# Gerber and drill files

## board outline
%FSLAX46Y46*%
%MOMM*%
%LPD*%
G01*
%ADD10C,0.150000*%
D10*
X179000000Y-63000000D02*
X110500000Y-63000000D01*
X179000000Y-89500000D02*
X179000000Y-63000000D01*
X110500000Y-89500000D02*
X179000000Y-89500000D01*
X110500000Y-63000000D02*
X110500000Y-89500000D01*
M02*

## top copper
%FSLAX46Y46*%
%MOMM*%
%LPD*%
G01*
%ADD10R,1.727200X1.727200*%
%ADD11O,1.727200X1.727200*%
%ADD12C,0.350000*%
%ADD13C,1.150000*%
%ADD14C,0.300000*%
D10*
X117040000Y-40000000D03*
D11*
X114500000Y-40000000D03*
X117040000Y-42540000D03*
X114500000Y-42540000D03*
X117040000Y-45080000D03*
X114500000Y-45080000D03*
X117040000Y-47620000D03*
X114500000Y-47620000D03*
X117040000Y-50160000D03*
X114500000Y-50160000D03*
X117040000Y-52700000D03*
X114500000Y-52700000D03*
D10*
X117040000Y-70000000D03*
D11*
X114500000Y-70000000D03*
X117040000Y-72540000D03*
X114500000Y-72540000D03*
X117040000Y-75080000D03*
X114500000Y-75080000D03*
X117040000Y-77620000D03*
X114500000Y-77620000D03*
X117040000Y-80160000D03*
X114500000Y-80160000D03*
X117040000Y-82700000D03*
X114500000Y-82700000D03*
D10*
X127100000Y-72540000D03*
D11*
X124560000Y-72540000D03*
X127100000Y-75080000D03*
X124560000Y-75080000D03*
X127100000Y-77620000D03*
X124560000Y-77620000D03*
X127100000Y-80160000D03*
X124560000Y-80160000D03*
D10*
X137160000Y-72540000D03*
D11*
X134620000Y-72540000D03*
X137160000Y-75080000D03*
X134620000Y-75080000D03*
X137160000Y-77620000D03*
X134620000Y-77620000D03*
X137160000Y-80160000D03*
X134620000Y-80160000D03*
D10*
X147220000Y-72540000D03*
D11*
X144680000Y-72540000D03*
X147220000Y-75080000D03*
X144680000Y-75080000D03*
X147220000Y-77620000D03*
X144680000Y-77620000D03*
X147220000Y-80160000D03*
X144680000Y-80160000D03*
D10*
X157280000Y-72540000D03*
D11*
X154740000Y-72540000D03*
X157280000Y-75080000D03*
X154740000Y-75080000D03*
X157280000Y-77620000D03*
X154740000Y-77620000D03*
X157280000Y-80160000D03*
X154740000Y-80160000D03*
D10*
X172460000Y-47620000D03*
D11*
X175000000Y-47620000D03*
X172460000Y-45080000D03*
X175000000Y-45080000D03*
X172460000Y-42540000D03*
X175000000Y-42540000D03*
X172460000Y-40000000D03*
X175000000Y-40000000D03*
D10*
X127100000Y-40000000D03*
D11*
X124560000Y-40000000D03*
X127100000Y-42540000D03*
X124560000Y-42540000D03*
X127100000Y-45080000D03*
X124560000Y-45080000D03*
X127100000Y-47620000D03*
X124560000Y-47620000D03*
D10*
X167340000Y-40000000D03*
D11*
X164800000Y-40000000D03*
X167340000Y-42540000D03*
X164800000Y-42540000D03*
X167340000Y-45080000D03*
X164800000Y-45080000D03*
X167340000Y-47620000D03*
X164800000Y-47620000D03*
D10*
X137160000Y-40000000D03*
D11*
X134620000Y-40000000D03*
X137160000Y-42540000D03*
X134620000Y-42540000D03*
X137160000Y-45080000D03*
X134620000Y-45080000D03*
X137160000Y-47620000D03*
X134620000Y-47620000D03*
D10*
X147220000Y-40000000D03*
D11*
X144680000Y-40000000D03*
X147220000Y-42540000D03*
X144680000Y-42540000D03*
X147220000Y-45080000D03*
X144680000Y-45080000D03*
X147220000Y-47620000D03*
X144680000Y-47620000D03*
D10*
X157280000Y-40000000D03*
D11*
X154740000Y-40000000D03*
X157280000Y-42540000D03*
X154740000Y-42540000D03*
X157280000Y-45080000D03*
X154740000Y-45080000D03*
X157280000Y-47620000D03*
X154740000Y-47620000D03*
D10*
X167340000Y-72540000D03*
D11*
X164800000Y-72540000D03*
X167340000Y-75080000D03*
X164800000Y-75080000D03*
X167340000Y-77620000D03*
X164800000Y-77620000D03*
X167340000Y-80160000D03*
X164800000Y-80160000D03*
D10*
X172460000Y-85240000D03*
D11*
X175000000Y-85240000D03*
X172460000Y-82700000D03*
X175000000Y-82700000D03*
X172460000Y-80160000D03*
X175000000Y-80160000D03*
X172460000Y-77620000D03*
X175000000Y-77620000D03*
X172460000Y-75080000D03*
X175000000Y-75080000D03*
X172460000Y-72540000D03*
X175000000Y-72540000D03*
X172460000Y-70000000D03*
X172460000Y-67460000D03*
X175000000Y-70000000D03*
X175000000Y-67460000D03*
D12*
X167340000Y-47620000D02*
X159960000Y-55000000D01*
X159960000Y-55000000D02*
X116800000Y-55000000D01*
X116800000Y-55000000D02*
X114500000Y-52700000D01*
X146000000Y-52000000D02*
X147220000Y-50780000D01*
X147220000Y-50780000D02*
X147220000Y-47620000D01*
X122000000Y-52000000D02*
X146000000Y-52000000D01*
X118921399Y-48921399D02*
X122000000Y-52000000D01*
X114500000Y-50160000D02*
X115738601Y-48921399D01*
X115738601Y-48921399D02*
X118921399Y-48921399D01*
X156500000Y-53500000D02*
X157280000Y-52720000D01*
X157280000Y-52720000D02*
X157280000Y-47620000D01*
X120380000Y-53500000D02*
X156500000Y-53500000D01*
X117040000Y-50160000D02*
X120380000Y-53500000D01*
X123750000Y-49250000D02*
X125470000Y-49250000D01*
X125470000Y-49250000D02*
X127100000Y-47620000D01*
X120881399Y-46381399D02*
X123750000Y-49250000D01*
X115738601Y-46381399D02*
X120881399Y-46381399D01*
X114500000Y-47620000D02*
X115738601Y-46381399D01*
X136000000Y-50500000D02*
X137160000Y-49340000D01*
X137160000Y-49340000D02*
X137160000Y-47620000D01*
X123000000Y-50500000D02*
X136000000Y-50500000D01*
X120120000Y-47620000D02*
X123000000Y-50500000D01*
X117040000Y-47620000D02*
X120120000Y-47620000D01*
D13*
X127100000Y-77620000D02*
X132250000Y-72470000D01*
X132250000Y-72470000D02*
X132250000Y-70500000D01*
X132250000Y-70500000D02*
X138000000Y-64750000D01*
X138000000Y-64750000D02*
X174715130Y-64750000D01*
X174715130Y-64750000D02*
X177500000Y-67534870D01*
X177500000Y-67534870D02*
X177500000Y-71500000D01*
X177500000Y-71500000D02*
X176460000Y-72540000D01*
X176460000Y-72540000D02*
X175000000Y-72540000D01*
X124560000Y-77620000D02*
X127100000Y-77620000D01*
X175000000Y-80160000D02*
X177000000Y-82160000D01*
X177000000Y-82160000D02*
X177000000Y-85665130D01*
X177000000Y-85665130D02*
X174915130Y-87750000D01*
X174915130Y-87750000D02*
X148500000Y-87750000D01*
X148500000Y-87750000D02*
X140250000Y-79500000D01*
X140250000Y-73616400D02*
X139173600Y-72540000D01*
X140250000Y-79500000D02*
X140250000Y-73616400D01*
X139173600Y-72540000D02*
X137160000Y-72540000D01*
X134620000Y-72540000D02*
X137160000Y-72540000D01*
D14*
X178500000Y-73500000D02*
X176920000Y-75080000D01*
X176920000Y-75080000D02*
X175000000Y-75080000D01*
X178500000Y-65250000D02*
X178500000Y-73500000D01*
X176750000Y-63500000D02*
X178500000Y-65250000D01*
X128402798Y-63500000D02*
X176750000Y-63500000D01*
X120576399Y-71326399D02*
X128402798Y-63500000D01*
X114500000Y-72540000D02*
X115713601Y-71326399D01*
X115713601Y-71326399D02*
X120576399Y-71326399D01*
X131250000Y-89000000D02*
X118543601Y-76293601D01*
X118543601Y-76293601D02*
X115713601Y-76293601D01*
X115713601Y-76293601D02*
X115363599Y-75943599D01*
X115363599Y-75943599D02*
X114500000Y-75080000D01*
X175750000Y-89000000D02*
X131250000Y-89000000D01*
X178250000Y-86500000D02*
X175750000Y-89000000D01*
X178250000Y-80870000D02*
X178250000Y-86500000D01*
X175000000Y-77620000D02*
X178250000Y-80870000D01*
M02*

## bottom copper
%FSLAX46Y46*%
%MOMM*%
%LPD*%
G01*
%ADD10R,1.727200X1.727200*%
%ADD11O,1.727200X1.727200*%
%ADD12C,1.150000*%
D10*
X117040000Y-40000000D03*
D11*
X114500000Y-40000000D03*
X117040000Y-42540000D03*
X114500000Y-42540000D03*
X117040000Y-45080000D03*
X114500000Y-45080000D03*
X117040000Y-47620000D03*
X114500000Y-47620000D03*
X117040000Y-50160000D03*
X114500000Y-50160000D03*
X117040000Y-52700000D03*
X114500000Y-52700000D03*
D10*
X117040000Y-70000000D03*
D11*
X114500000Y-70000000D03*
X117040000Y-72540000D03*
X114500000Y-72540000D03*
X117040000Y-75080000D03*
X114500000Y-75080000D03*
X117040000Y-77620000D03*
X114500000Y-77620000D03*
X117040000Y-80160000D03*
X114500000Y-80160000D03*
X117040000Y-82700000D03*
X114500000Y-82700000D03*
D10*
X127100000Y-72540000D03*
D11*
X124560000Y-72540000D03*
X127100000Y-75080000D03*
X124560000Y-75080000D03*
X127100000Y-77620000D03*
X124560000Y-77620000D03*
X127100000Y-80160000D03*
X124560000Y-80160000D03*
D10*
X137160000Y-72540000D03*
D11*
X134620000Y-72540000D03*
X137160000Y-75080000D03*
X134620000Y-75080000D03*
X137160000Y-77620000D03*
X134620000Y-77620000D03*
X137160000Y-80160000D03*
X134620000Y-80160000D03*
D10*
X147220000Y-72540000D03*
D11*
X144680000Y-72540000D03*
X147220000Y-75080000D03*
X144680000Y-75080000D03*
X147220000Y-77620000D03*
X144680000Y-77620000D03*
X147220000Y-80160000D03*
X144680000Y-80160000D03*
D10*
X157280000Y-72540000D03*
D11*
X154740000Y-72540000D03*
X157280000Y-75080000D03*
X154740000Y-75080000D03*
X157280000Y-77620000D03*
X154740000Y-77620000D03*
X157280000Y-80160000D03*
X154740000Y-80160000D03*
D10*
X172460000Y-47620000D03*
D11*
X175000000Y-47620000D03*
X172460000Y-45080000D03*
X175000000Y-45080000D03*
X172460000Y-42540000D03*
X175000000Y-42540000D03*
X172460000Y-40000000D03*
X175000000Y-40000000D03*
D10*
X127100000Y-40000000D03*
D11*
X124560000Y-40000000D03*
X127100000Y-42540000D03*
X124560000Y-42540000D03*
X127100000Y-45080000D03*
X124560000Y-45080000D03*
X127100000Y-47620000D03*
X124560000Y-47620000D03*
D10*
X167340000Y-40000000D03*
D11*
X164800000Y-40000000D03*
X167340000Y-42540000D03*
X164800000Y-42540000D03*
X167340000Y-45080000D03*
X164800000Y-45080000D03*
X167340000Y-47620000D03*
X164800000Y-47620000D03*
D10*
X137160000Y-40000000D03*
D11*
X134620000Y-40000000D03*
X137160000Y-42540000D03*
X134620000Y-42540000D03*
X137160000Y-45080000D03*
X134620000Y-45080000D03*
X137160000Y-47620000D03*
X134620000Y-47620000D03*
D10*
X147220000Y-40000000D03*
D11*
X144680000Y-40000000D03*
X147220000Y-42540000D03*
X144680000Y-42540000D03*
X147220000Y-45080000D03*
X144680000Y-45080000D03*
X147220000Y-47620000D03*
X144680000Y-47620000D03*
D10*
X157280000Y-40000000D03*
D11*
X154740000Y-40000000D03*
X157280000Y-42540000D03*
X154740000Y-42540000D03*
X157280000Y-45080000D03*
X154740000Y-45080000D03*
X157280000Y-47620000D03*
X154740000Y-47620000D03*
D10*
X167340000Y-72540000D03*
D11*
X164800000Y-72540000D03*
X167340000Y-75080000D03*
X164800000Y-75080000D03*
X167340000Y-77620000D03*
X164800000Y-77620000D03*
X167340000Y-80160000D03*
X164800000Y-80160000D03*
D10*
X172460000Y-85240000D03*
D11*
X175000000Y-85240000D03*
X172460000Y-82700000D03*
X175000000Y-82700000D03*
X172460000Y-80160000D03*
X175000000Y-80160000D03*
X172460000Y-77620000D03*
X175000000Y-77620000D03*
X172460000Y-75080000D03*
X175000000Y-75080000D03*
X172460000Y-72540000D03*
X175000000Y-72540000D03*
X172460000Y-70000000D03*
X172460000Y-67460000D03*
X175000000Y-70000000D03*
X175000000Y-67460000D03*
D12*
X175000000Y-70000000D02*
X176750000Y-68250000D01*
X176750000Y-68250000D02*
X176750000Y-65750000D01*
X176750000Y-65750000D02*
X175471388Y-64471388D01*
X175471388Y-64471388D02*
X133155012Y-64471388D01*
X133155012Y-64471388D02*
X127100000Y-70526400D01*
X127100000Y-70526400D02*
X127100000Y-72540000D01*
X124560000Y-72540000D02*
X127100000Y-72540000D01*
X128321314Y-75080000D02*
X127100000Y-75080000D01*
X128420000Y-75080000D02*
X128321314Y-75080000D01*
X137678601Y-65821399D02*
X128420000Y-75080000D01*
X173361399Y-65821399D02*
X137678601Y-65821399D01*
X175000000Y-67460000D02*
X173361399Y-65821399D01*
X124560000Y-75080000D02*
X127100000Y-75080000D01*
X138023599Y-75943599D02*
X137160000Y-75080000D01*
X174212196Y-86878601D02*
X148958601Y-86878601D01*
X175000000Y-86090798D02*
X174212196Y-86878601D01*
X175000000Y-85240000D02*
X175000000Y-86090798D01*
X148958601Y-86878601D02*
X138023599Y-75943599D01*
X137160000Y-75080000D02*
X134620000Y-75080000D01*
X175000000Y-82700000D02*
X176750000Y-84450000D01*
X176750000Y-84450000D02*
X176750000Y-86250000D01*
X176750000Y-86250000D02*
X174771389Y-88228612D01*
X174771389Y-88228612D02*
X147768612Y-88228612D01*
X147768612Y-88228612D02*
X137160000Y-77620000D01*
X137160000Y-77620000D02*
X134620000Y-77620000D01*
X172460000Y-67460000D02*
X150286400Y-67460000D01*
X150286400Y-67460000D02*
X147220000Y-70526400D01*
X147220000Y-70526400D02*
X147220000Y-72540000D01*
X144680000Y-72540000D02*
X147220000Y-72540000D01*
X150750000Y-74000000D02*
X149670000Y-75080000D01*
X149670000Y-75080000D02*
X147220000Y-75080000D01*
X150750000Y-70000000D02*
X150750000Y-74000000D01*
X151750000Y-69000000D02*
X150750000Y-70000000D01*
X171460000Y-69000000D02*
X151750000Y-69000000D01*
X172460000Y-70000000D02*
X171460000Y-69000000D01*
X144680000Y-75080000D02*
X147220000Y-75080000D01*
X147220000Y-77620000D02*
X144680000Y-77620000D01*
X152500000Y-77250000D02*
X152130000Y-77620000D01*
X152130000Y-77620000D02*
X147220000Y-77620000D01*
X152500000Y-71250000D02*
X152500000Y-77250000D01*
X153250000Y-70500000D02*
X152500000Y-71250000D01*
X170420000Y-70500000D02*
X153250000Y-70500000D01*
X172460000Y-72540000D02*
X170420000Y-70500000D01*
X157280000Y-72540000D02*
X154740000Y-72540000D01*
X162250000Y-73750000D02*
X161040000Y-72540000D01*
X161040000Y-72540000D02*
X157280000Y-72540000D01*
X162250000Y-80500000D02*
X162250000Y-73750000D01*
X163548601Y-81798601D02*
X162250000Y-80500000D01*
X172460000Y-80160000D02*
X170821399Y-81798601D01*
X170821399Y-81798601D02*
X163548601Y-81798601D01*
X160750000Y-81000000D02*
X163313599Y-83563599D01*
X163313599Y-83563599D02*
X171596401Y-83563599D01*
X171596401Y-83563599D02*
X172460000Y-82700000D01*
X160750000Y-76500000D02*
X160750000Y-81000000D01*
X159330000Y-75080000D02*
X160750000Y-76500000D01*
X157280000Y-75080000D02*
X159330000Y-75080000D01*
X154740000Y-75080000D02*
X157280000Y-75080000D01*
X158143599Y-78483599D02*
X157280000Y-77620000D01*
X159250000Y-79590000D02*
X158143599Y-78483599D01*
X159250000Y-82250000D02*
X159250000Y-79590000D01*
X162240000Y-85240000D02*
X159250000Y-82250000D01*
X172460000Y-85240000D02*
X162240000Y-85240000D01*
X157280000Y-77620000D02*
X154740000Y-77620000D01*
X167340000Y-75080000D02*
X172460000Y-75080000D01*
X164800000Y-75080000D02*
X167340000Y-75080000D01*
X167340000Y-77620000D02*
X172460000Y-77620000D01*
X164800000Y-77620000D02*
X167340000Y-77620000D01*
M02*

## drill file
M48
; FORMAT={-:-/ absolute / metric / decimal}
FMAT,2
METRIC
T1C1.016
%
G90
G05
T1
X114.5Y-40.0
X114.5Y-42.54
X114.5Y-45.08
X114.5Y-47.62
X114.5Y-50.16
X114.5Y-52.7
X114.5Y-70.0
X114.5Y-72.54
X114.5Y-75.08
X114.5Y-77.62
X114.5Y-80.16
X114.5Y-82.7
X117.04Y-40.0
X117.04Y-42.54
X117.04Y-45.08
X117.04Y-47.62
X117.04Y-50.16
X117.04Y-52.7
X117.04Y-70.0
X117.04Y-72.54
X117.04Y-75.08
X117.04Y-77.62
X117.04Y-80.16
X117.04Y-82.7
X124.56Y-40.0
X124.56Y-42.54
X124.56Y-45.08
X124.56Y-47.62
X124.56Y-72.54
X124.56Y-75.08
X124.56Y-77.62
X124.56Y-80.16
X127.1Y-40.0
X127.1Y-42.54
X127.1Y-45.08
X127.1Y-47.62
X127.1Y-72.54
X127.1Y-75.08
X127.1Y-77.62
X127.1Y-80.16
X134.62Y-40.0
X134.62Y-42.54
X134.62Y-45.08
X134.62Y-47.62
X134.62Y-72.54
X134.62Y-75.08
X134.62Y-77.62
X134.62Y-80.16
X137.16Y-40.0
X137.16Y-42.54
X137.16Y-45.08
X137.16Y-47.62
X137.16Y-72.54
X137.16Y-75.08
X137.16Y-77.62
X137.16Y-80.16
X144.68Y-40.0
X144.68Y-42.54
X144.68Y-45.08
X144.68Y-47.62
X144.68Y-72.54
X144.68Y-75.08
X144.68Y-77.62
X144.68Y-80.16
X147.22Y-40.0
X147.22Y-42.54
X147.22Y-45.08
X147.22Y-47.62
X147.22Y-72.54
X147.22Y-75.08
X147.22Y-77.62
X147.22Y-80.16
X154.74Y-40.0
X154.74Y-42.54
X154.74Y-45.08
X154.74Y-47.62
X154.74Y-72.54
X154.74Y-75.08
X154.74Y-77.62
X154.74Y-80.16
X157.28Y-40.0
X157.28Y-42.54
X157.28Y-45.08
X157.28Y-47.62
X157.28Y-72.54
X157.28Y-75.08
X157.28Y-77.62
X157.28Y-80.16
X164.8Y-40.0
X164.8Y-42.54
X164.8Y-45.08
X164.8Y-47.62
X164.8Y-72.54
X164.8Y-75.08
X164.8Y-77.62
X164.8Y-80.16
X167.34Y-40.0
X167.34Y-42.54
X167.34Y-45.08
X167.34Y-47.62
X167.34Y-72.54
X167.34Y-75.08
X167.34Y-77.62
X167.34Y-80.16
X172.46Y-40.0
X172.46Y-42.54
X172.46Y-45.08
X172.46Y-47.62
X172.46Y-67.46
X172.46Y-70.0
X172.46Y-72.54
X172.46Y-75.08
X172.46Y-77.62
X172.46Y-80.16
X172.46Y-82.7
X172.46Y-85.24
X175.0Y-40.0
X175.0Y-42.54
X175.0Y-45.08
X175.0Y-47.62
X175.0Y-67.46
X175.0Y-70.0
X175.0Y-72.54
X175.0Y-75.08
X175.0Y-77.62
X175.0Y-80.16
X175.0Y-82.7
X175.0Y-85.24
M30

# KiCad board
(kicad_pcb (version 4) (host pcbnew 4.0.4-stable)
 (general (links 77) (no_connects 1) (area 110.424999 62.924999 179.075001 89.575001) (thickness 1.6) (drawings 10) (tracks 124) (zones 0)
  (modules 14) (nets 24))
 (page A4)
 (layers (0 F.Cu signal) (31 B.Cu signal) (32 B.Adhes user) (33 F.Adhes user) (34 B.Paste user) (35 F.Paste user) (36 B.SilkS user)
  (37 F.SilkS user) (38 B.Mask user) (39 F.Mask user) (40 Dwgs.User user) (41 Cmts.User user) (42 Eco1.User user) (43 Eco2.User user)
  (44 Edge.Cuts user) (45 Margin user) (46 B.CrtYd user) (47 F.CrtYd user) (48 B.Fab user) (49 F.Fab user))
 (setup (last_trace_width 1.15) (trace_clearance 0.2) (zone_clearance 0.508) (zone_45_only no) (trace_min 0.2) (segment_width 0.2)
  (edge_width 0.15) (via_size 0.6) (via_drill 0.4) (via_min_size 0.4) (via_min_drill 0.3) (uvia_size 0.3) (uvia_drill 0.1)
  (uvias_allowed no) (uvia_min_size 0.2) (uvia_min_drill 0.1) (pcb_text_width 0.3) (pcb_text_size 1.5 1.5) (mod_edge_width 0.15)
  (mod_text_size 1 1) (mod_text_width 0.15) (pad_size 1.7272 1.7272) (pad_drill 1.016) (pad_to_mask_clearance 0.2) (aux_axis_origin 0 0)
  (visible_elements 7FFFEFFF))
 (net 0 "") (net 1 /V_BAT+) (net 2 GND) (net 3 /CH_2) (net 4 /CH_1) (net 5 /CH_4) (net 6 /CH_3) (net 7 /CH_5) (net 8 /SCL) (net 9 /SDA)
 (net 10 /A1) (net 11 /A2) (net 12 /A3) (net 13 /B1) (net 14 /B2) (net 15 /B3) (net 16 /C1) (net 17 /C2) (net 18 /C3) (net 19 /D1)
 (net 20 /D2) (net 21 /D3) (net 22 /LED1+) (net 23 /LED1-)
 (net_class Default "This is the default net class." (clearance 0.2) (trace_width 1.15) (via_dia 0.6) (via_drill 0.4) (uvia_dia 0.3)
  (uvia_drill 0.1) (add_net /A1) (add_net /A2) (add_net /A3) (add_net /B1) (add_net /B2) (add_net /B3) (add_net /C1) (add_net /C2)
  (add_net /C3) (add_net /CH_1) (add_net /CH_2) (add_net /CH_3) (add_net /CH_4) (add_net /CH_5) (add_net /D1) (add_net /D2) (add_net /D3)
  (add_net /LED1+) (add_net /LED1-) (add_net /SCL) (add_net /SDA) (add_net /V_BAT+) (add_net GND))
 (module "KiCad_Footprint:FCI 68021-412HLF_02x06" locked (layer F.Cu) (at 117.04 40 270)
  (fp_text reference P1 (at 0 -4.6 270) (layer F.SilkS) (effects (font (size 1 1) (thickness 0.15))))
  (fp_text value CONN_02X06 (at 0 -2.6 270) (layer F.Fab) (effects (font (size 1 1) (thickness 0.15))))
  (pad 1 thru_hole rect (at 0 0 270) (size 1.7272 1.7272) (drill 1.016) (layers *.Cu *.Mask F.SilkS) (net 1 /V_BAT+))
  (pad 2 thru_hole oval (at 0 2.54 270) (size 1.7272 1.7272) (drill 1.016) (layers *.Cu *.Mask F.SilkS) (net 1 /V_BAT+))
  (pad 3 thru_hole oval (at 2.54 0 270) (size 1.7272 1.7272) (drill 1.016) (layers *.Cu *.Mask F.SilkS) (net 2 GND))
  (pad 4 thru_hole oval (at 2.54 2.54 270) (size 1.7272 1.7272) (drill 1.016) (layers *.Cu *.Mask F.SilkS) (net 2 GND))
  (pad 5 thru_hole oval (at 5.08 0 270) (size 1.7272 1.7272) (drill 1.016) (layers *.Cu *.Mask F.SilkS) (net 2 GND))
  (pad 6 thru_hole oval (at 5.08 2.54 270) (size 1.7272 1.7272) (drill 1.016) (layers *.Cu *.Mask F.SilkS) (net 2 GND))
  (pad 7 thru_hole oval (at 7.62 0 270) (size 1.7272 1.7272) (drill 1.016) (layers *.Cu *.Mask F.SilkS) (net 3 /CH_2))
  (pad 8 thru_hole oval (at 7.62 2.54 270) (size 1.7272 1.7272) (drill 1.016) (layers *.Cu *.Mask F.SilkS) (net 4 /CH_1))
  (pad 9 thru_hole oval (at 10.16 0 270) (size 1.7272 1.7272) (drill 1.016) (layers *.Cu *.Mask F.SilkS) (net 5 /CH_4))
  (pad 10 thru_hole oval (at 10.16 2.54 270) (size 1.7272 1.7272) (drill 1.016) (layers *.Cu *.Mask F.SilkS) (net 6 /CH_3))
  (pad 11 thru_hole oval (at 12.7 0 270) (size 1.7272 1.7272) (drill 1.016) (layers *.Cu *.Mask F.SilkS))
  (pad 12 thru_hole oval (at 12.7 2.54 270) (size 1.7272 1.7272) (drill 1.016) (layers *.Cu *.Mask F.SilkS) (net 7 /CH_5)))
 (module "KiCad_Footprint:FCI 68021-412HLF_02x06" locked (layer F.Cu) (at 117.04 70 270)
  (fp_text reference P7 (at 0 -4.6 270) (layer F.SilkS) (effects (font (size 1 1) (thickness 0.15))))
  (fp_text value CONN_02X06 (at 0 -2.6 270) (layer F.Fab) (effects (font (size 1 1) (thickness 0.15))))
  (pad 1 thru_hole rect (at 0 0 270) (size 1.7272 1.7272) (drill 1.016) (layers *.Cu *.Mask F.SilkS))
  (pad 2 thru_hole oval (at 0 2.54 270) (size 1.7272 1.7272) (drill 1.016) (layers *.Cu *.Mask F.SilkS))
  (pad 3 thru_hole oval (at 2.54 0 270) (size 1.7272 1.7272) (drill 1.016) (layers *.Cu *.Mask F.SilkS))
  (pad 4 thru_hole oval (at 2.54 2.54 270) (size 1.7272 1.7272) (drill 1.016) (layers *.Cu *.Mask F.SilkS) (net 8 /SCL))
  (pad 5 thru_hole oval (at 5.08 0 270) (size 1.7272 1.7272) (drill 1.016) (layers *.Cu *.Mask F.SilkS))
  (pad 6 thru_hole oval (at 5.08 2.54 270) (size 1.7272 1.7272) (drill 1.016) (layers *.Cu *.Mask F.SilkS) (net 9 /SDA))
  (pad 7 thru_hole oval (at 7.62 0 270) (size 1.7272 1.7272) (drill 1.016) (layers *.Cu *.Mask F.SilkS))
  (pad 8 thru_hole oval (at 7.62 2.54 270) (size 1.7272 1.7272) (drill 1.016) (layers *.Cu *.Mask F.SilkS))
  (pad 9 thru_hole oval (at 10.16 0 270) (size 1.7272 1.7272) (drill 1.016) (layers *.Cu *.Mask F.SilkS))
  (pad 10 thru_hole oval (at 10.16 2.54 270) (size 1.7272 1.7272) (drill 1.016) (layers *.Cu *.Mask F.SilkS))
  (pad 11 thru_hole oval (at 12.7 0 270) (size 1.7272 1.7272) (drill 1.016) (layers *.Cu *.Mask F.SilkS))
  (pad 12 thru_hole oval (at 12.7 2.54 270) (size 1.7272 1.7272) (drill 1.016) (layers *.Cu *.Mask F.SilkS)))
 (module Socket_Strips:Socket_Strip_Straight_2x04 (layer F.Cu) (at 127.1 72.54 270)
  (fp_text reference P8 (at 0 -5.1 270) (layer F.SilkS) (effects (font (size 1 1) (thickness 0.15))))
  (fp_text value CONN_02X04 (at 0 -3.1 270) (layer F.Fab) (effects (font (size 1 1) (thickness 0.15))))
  (pad 1 thru_hole rect (at 0 0 270) (size 1.7272 1.7272) (drill 1.016) (layers *.Cu *.Mask F.SilkS) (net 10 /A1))
  (pad 2 thru_hole oval (at 0 2.54 270) (size 1.7272 1.7272) (drill 1.016) (layers *.Cu *.Mask F.SilkS) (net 10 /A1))
  (pad 3 thru_hole oval (at 2.54 0 270) (size 1.7272 1.7272) (drill 1.016) (layers *.Cu *.Mask F.SilkS) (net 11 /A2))
  (pad 4 thru_hole oval (at 2.54 2.54 270) (size 1.7272 1.7272) (drill 1.016) (layers *.Cu *.Mask F.SilkS) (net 11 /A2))
  (pad 5 thru_hole oval (at 5.08 0 270) (size 1.7272 1.7272) (drill 1.016) (layers *.Cu *.Mask F.SilkS) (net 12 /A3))
  (pad 6 thru_hole oval (at 5.08 2.54 270) (size 1.7272 1.7272) (drill 1.016) (layers *.Cu *.Mask F.SilkS) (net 12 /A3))
  (pad 7 thru_hole oval (at 7.62 0 270) (size 1.7272 1.7272) (drill 1.016) (layers *.Cu *.Mask F.SilkS))
  (pad 8 thru_hole oval (at 7.62 2.54 270) (size 1.7272 1.7272) (drill 1.016) (layers *.Cu *.Mask F.SilkS)))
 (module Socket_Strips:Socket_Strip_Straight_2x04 (layer F.Cu) (at 137.16 72.54 270)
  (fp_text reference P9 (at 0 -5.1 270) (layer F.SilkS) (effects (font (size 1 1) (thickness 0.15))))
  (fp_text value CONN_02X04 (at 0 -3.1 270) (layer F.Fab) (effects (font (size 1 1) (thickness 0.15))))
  (pad 1 thru_hole rect (at 0 0 270) (size 1.7272 1.7272) (drill 1.016) (layers *.Cu *.Mask F.SilkS) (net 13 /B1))
  (pad 2 thru_hole oval (at 0 2.54 270) (size 1.7272 1.7272) (drill 1.016) (layers *.Cu *.Mask F.SilkS) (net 13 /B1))
  (pad 3 thru_hole oval (at 2.54 0 270) (size 1.7272 1.7272) (drill 1.016) (layers *.Cu *.Mask F.SilkS) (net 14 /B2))
  (pad 4 thru_hole oval (at 2.54 2.54 270) (size 1.7272 1.7272) (drill 1.016) (layers *.Cu *.Mask F.SilkS) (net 14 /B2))
  (pad 5 thru_hole oval (at 5.08 0 270) (size 1.7272 1.7272) (drill 1.016) (layers *.Cu *.Mask F.SilkS) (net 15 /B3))
  (pad 6 thru_hole oval (at 5.08 2.54 270) (size 1.7272 1.7272) (drill 1.016) (layers *.Cu *.Mask F.SilkS) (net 15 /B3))
  (pad 7 thru_hole oval (at 7.62 0 270) (size 1.7272 1.7272) (drill 1.016) (layers *.Cu *.Mask F.SilkS))
  (pad 8 thru_hole oval (at 7.62 2.54 270) (size 1.7272 1.7272) (drill 1.016) (layers *.Cu *.Mask F.SilkS)))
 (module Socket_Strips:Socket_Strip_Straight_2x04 (layer F.Cu) (at 147.22 72.54 270)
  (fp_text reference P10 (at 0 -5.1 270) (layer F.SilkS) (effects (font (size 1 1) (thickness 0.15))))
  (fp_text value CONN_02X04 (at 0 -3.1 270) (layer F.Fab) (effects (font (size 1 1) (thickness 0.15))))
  (pad 1 thru_hole rect (at 0 0 270) (size 1.7272 1.7272) (drill 1.016) (layers *.Cu *.Mask F.SilkS) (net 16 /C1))
  (pad 2 thru_hole oval (at 0 2.54 270) (size 1.7272 1.7272) (drill 1.016) (layers *.Cu *.Mask F.SilkS) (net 16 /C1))
  (pad 3 thru_hole oval (at 2.54 0 270) (size 1.7272 1.7272) (drill 1.016) (layers *.Cu *.Mask F.SilkS) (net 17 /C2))
  (pad 4 thru_hole oval (at 2.54 2.54 270) (size 1.7272 1.7272) (drill 1.016) (layers *.Cu *.Mask F.SilkS) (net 17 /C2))
  (pad 5 thru_hole oval (at 5.08 0 270) (size 1.7272 1.7272) (drill 1.016) (layers *.Cu *.Mask F.SilkS) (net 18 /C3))
  (pad 6 thru_hole oval (at 5.08 2.54 270) (size 1.7272 1.7272) (drill 1.016) (layers *.Cu *.Mask F.SilkS) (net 18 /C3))
  (pad 7 thru_hole oval (at 7.62 0 270) (size 1.7272 1.7272) (drill 1.016) (layers *.Cu *.Mask F.SilkS))
  (pad 8 thru_hole oval (at 7.62 2.54 270) (size 1.7272 1.7272) (drill 1.016) (layers *.Cu *.Mask F.SilkS)))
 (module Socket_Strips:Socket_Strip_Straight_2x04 (layer F.Cu) (at 157.28 72.54 270)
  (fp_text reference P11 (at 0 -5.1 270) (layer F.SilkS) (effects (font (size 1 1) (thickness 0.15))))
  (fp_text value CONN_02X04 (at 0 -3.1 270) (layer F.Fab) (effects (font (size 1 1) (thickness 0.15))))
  (pad 1 thru_hole rect (at 0 0 270) (size 1.7272 1.7272) (drill 1.016) (layers *.Cu *.Mask F.SilkS) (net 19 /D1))
  (pad 2 thru_hole oval (at 0 2.54 270) (size 1.7272 1.7272) (drill 1.016) (layers *.Cu *.Mask F.SilkS) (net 19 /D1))
  (pad 3 thru_hole oval (at 2.54 0 270) (size 1.7272 1.7272) (drill 1.016) (layers *.Cu *.Mask F.SilkS) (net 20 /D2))
  (pad 4 thru_hole oval (at 2.54 2.54 270) (size 1.7272 1.7272) (drill 1.016) (layers *.Cu *.Mask F.SilkS) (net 20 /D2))
  (pad 5 thru_hole oval (at 5.08 0 270) (size 1.7272 1.7272) (drill 1.016) (layers *.Cu *.Mask F.SilkS) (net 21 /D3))
  (pad 6 thru_hole oval (at 5.08 2.54 270) (size 1.7272 1.7272) (drill 1.016) (layers *.Cu *.Mask F.SilkS) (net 21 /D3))
  (pad 7 thru_hole oval (at 7.62 0 270) (size 1.7272 1.7272) (drill 1.016) (layers *.Cu *.Mask F.SilkS))
  (pad 8 thru_hole oval (at 7.62 2.54 270) (size 1.7272 1.7272) (drill 1.016) (layers *.Cu *.Mask F.SilkS)))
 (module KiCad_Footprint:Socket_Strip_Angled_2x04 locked (layer F.Cu) (at 172.46 47.62 90)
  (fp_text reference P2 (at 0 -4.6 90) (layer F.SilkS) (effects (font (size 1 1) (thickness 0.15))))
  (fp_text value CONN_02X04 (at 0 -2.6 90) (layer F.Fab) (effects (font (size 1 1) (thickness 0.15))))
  (pad 1 thru_hole rect (at 0 0 90) (size 1.7272 1.7272) (drill 1.016) (layers *.Cu *.Mask F.SilkS) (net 2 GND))
  (pad 2 thru_hole oval (at 0 2.54 90) (size 1.7272 1.7272) (drill 1.016) (layers *.Cu *.Mask F.SilkS) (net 2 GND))
  (pad 3 thru_hole oval (at 2.54 0 90) (size 1.7272 1.7272) (drill 1.016) (layers *.Cu *.Mask F.SilkS) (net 2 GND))
  (pad 4 thru_hole oval (at 2.54 2.54 90) (size 1.7272 1.7272) (drill 1.016) (layers *.Cu *.Mask F.SilkS) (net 2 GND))
  (pad 5 thru_hole oval (at 5.08 0 90) (size 1.7272 1.7272) (drill 1.016) (layers *.Cu *.Mask F.SilkS) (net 1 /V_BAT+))
  (pad 6 thru_hole oval (at 5.08 2.54 90) (size 1.7272 1.7272) (drill 1.016) (layers *.Cu *.Mask F.SilkS) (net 1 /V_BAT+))
  (pad 7 thru_hole oval (at 7.62 0 90) (size 1.7272 1.7272) (drill 1.016) (layers *.Cu *.Mask F.SilkS) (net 1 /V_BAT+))
  (pad 8 thru_hole oval (at 7.62 2.54 90) (size 1.7272 1.7272) (drill 1.016) (layers *.Cu *.Mask F.SilkS) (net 1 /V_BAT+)))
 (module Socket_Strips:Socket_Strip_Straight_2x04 (layer F.Cu) (at 127.1 40 270)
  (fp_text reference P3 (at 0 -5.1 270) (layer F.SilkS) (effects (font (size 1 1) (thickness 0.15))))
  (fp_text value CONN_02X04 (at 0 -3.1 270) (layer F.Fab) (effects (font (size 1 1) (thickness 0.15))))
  (pad 1 thru_hole rect (at 0 0 270) (size 1.7272 1.7272) (drill 1.016) (layers *.Cu *.Mask F.SilkS) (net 1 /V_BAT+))
  (pad 2 thru_hole oval (at 0 2.54 270) (size 1.7272 1.7272) (drill 1.016) (layers *.Cu *.Mask F.SilkS) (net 1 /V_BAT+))
  (pad 3 thru_hole oval (at 2.54 0 270) (size 1.7272 1.7272) (drill 1.016) (layers *.Cu *.Mask F.SilkS) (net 2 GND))
  (pad 4 thru_hole oval (at 2.54 2.54 270) (size 1.7272 1.7272) (drill 1.016) (layers *.Cu *.Mask F.SilkS) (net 2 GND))
  (pad 5 thru_hole oval (at 5.08 0 270) (size 1.7272 1.7272) (drill 1.016) (layers *.Cu *.Mask F.SilkS) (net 2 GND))
  (pad 6 thru_hole oval (at 5.08 2.54 270) (size 1.7272 1.7272) (drill 1.016) (layers *.Cu *.Mask F.SilkS) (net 2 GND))
  (pad 7 thru_hole oval (at 7.62 0 270) (size 1.7272 1.7272) (drill 1.016) (layers *.Cu *.Mask F.SilkS) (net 4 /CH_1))
  (pad 8 thru_hole oval (at 7.62 2.54 270) (size 1.7272 1.7272) (drill 1.016) (layers *.Cu *.Mask F.SilkS)))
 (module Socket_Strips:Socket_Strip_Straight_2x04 (layer F.Cu) (at 167.34 40 270)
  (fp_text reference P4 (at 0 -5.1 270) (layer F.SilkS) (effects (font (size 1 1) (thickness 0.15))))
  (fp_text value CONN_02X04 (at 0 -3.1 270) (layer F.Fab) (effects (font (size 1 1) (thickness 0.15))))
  (pad 1 thru_hole rect (at 0 0 270) (size 1.7272 1.7272) (drill 1.016) (layers *.Cu *.Mask F.SilkS) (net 1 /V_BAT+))
  (pad 2 thru_hole oval (at 0 2.54 270) (size 1.7272 1.7272) (drill 1.016) (layers *.Cu *.Mask F.SilkS) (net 1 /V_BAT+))
  (pad 3 thru_hole oval (at 2.54 0 270) (size 1.7272 1.7272) (drill 1.016) (layers *.Cu *.Mask F.SilkS) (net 2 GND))
  (pad 4 thru_hole oval (at 2.54 2.54 270) (size 1.7272 1.7272) (drill 1.016) (layers *.Cu *.Mask F.SilkS) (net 2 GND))
  (pad 5 thru_hole oval (at 5.08 0 270) (size 1.7272 1.7272) (drill 1.016) (layers *.Cu *.Mask F.SilkS) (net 2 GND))
  (pad 6 thru_hole oval (at 5.08 2.54 270) (size 1.7272 1.7272) (drill 1.016) (layers *.Cu *.Mask F.SilkS) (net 2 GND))
  (pad 7 thru_hole oval (at 7.62 0 270) (size 1.7272 1.7272) (drill 1.016) (layers *.Cu *.Mask F.SilkS) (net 7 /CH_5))
  (pad 8 thru_hole oval (at 7.62 2.54 270) (size 1.7272 1.7272) (drill 1.016) (layers *.Cu *.Mask F.SilkS)))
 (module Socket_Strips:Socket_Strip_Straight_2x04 (layer F.Cu) (at 137.16 40 270)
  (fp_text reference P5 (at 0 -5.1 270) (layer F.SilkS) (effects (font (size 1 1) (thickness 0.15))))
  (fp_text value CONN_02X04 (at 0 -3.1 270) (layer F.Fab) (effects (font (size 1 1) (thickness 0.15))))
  (pad 1 thru_hole rect (at 0 0 270) (size 1.7272 1.7272) (drill 1.016) (layers *.Cu *.Mask F.SilkS) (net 1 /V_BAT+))
  (pad 2 thru_hole oval (at 0 2.54 270) (size 1.7272 1.7272) (drill 1.016) (layers *.Cu *.Mask F.SilkS) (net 1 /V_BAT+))
  (pad 3 thru_hole oval (at 2.54 0 270) (size 1.7272 1.7272) (drill 1.016) (layers *.Cu *.Mask F.SilkS) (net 2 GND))
  (pad 4 thru_hole oval (at 2.54 2.54 270) (size 1.7272 1.7272) (drill 1.016) (layers *.Cu *.Mask F.SilkS) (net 2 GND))
  (pad 5 thru_hole oval (at 5.08 0 270) (size 1.7272 1.7272) (drill 1.016) (layers *.Cu *.Mask F.SilkS) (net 2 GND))
  (pad 6 thru_hole oval (at 5.08 2.54 270) (size 1.7272 1.7272) (drill 1.016) (layers *.Cu *.Mask F.SilkS) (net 2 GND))
  (pad 7 thru_hole oval (at 7.62 0 270) (size 1.7272 1.7272) (drill 1.016) (layers *.Cu *.Mask F.SilkS) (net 3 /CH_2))
  (pad 8 thru_hole oval (at 7.62 2.54 270) (size 1.7272 1.7272) (drill 1.016) (layers *.Cu *.Mask F.SilkS)))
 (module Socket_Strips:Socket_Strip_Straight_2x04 (layer F.Cu) (at 147.22 40 270)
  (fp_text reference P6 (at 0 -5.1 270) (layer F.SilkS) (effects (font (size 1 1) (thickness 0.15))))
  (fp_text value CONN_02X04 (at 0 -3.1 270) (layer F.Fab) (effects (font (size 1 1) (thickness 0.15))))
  (pad 1 thru_hole rect (at 0 0 270) (size 1.7272 1.7272) (drill 1.016) (layers *.Cu *.Mask F.SilkS) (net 1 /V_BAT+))
  (pad 2 thru_hole oval (at 0 2.54 270) (size 1.7272 1.7272) (drill 1.016) (layers *.Cu *.Mask F.SilkS) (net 1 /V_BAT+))
  (pad 3 thru_hole oval (at 2.54 0 270) (size 1.7272 1.7272) (drill 1.016) (layers *.Cu *.Mask F.SilkS) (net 2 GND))
  (pad 4 thru_hole oval (at 2.54 2.54 270) (size 1.7272 1.7272) (drill 1.016) (layers *.Cu *.Mask F.SilkS) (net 2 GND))
  (pad 5 thru_hole oval (at 5.08 0 270) (size 1.7272 1.7272) (drill 1.016) (layers *.Cu *.Mask F.SilkS) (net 2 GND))
  (pad 6 thru_hole oval (at 5.08 2.54 270) (size 1.7272 1.7272) (drill 1.016) (layers *.Cu *.Mask F.SilkS) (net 2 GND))
  (pad 7 thru_hole oval (at 7.62 0 270) (size 1.7272 1.7272) (drill 1.016) (layers *.Cu *.Mask F.SilkS) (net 6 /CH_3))
  (pad 8 thru_hole oval (at 7.62 2.54 270) (size 1.7272 1.7272) (drill 1.016) (layers *.Cu *.Mask F.SilkS)))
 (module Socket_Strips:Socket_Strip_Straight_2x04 (layer F.Cu) (at 157.28 40 270)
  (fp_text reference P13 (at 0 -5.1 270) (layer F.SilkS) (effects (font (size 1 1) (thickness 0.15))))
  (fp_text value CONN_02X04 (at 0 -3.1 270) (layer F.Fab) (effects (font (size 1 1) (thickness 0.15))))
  (pad 1 thru_hole rect (at 0 0 270) (size 1.7272 1.7272) (drill 1.016) (layers *.Cu *.Mask F.SilkS) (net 1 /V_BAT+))
  (pad 2 thru_hole oval (at 0 2.54 270) (size 1.7272 1.7272) (drill 1.016) (layers *.Cu *.Mask F.SilkS) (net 1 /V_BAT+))
  (pad 3 thru_hole oval (at 2.54 0 270) (size 1.7272 1.7272) (drill 1.016) (layers *.Cu *.Mask F.SilkS) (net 2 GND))
  (pad 4 thru_hole oval (at 2.54 2.54 270) (size 1.7272 1.7272) (drill 1.016) (layers *.Cu *.Mask F.SilkS) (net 2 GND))
  (pad 5 thru_hole oval (at 5.08 0 270) (size 1.7272 1.7272) (drill 1.016) (layers *.Cu *.Mask F.SilkS) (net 2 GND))
  (pad 6 thru_hole oval (at 5.08 2.54 270) (size 1.7272 1.7272) (drill 1.016) (layers *.Cu *.Mask F.SilkS) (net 2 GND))
  (pad 7 thru_hole oval (at 7.62 0 270) (size 1.7272 1.7272) (drill 1.016) (layers *.Cu *.Mask F.SilkS) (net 5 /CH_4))
  (pad 8 thru_hole oval (at 7.62 2.54 270) (size 1.7272 1.7272) (drill 1.016) (layers *.Cu *.Mask F.SilkS)))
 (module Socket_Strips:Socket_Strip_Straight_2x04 (layer F.Cu) (at 167.34 72.54 270)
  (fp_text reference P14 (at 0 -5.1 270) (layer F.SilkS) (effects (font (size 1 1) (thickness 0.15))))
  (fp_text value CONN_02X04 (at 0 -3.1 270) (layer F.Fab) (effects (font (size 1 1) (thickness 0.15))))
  (pad 1 thru_hole rect (at 0 0 270) (size 1.7272 1.7272) (drill 1.016) (layers *.Cu *.Mask F.SilkS))
  (pad 2 thru_hole oval (at 0 2.54 270) (size 1.7272 1.7272) (drill 1.016) (layers *.Cu *.Mask F.SilkS))
  (pad 3 thru_hole oval (at 2.54 0 270) (size 1.7272 1.7272) (drill 1.016) (layers *.Cu *.Mask F.SilkS) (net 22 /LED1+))
  (pad 4 thru_hole oval (at 2.54 2.54 270) (size 1.7272 1.7272) (drill 1.016) (layers *.Cu *.Mask F.SilkS) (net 22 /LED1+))
  (pad 5 thru_hole oval (at 5.08 0 270) (size 1.7272 1.7272) (drill 1.016) (layers *.Cu *.Mask F.SilkS) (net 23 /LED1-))
  (pad 6 thru_hole oval (at 5.08 2.54 270) (size 1.7272 1.7272) (drill 1.016) (layers *.Cu *.Mask F.SilkS) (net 23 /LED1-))
  (pad 7 thru_hole oval (at 7.62 0 270) (size 1.7272 1.7272) (drill 1.016) (layers *.Cu *.Mask F.SilkS))
  (pad 8 thru_hole oval (at 7.62 2.54 270) (size 1.7272 1.7272) (drill 1.016) (layers *.Cu *.Mask F.SilkS)))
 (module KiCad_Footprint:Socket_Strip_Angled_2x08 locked (layer F.Cu) (at 172.46 85.24 90)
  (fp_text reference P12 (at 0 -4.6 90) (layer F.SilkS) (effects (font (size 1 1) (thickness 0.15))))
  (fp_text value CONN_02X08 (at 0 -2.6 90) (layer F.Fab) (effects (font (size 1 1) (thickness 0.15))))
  (pad 1 thru_hole rect (at 0 0 90) (size 1.7272 1.7272) (drill 1.016) (layers *.Cu *.Mask F.SilkS) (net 21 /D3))
  (pad 2 thru_hole oval (at 0 2.54 90) (size 1.7272 1.7272) (drill 1.016) (layers *.Cu *.Mask F.SilkS) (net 14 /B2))
  (pad 3 thru_hole oval (at 2.54 0 90) (size 1.7272 1.7272) (drill 1.016) (layers *.Cu *.Mask F.SilkS) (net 20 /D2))
  (pad 4 thru_hole oval (at 2.54 2.54 90) (size 1.7272 1.7272) (drill 1.016) (layers *.Cu *.Mask F.SilkS) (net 15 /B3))
  (pad 5 thru_hole oval (at 5.08 0 90) (size 1.7272 1.7272) (drill 1.016) (layers *.Cu *.Mask F.SilkS) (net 19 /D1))
  (pad 6 thru_hole oval (at 5.08 2.54 90) (size 1.7272 1.7272) (drill 1.016) (layers *.Cu *.Mask F.SilkS) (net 13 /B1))
  (pad 7 thru_hole oval (at 7.62 0 90) (size 1.7272 1.7272) (drill 1.016) (layers *.Cu *.Mask F.SilkS) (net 23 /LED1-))
  (pad 8 thru_hole oval (at 7.62 2.54 90) (size 1.7272 1.7272) (drill 1.016) (layers *.Cu *.Mask F.SilkS) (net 9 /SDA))
  (pad 9 thru_hole oval (at 10.16 0 90) (size 1.7272 1.7272) (drill 1.016) (layers *.Cu *.Mask F.SilkS) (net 22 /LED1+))
  (pad 10 thru_hole oval (at 10.16 2.54 90) (size 1.7272 1.7272) (drill 1.016) (layers *.Cu *.Mask F.SilkS) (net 8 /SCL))
  (pad 11 thru_hole oval (at 12.7 0 90) (size 1.7272 1.7272) (drill 1.016) (layers *.Cu *.Mask F.SilkS) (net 18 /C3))
  (pad 12 thru_hole oval (at 12.7 2.54 90) (size 1.7272 1.7272) (drill 1.016) (layers *.Cu *.Mask F.SilkS) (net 12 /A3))
  (pad 13 thru_hole oval (at 15.24 0 90) (size 1.7272 1.7272) (drill 1.016) (layers *.Cu *.Mask F.SilkS) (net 17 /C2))
  (pad 15 thru_hole oval (at 17.78 0 90) (size 1.7272 1.7272) (drill 1.016) (layers *.Cu *.Mask F.SilkS) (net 16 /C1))
  (pad 14 thru_hole oval (at 15.24 2.54 90) (size 1.7272 1.7272) (drill 1.016) (layers *.Cu *.Mask F.SilkS) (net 10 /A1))
  (pad 16 thru_hole oval (at 17.78 2.54 90) (size 1.7272 1.7272) (drill 1.016) (layers *.Cu *.Mask F.SilkS) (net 11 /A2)))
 (gr_line (start 179 63) (end 110.5 63) (layer Edge.Cuts) (width 0.15))
 (gr_line (start 179 89.5) (end 179 63) (layer Edge.Cuts) (width 0.15))
 (gr_line (start 110.5 89.5) (end 179 89.5) (layer Edge.Cuts) (width 0.15))
 (gr_line (start 110.5 63) (end 110.5 89.5) (layer Edge.Cuts) (width 0.15))
 (segment (start 167.34 47.62) (end 159.96 55) (width 0.35) (layer F.Cu) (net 7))
 (segment (start 159.96 55) (end 116.8 55) (width 0.35) (layer F.Cu) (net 7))
 (segment (start 116.8 55) (end 114.5 52.7) (width 0.35) (layer F.Cu) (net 7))
 (segment (start 146 52) (end 147.22 50.78) (width 0.35) (layer F.Cu) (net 6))
 (segment (start 147.22 50.78) (end 147.22 47.62) (width 0.35) (layer F.Cu) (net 6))
 (segment (start 122 52) (end 146 52) (width 0.35) (layer F.Cu) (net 6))
 (segment (start 118.921399 48.921399) (end 122 52) (width 0.35) (layer F.Cu) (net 6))
 (segment (start 114.5 50.16) (end 115.738601 48.921399) (width 0.35) (layer F.Cu) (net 6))
 (segment (start 115.738601 48.921399) (end 118.921399 48.921399) (width 0.35) (layer F.Cu) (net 6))
 (segment (start 156.5 53.5) (end 157.28 52.72) (width 0.35) (layer F.Cu) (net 5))
 (segment (start 157.28 52.72) (end 157.28 47.62) (width 0.35) (layer F.Cu) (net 5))
 (segment (start 120.38 53.5) (end 156.5 53.5) (width 0.35) (layer F.Cu) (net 5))
 (segment (start 117.04 50.16) (end 120.38 53.5) (width 0.35) (layer F.Cu) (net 5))
 (segment (start 123.75 49.25) (end 125.47 49.25) (width 0.35) (layer F.Cu) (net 4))
 (segment (start 125.47 49.25) (end 127.1 47.62) (width 0.35) (layer F.Cu) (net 4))
 (segment (start 120.881399 46.381399) (end 123.75 49.25) (width 0.35) (layer F.Cu) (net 4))
 (segment (start 115.738601 46.381399) (end 120.881399 46.381399) (width 0.35) (layer F.Cu) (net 4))
 (segment (start 114.5 47.62) (end 115.738601 46.381399) (width 0.35) (layer F.Cu) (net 4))
 (segment (start 136 50.5) (end 137.16 49.34) (width 0.35) (layer F.Cu) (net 3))
 (segment (start 137.16 49.34) (end 137.16 47.62) (width 0.35) (layer F.Cu) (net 3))
 (segment (start 123 50.5) (end 136 50.5) (width 0.35) (layer F.Cu) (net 3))
 (segment (start 120.12 47.62) (end 123 50.5) (width 0.35) (layer F.Cu) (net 3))
 (segment (start 117.04 47.62) (end 120.12 47.62) (width 0.35) (layer F.Cu) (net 3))
 (segment (start 175 70) (end 176.75 68.25) (width 1.15) (layer B.Cu) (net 10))
 (segment (start 176.75 68.25) (end 176.75 65.75) (width 1.15) (layer B.Cu) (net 10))
 (segment (start 176.75 65.75) (end 175.471388 64.471388) (width 1.15) (layer B.Cu) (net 10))
 (segment (start 175.471388 64.471388) (end 133.155012 64.471388) (width 1.15) (layer B.Cu) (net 10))
 (segment (start 133.155012 64.471388) (end 127.1 70.5264) (width 1.15) (layer B.Cu) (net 10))
 (segment (start 127.1 70.5264) (end 127.1 72.54) (width 1.15) (layer B.Cu) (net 10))
 (segment (start 124.56 72.54) (end 127.1 72.54) (width 1.15) (layer B.Cu) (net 10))
 (segment (start 128.321314 75.08) (end 127.1 75.08) (width 1.15) (layer B.Cu) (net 11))
 (segment (start 128.42 75.08) (end 128.321314 75.08) (width 1.15) (layer B.Cu) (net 11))
 (segment (start 137.678601 65.821399) (end 128.42 75.08) (width 1.15) (layer B.Cu) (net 11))
 (segment (start 173.361399 65.821399) (end 137.678601 65.821399) (width 1.15) (layer B.Cu) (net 11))
 (segment (start 175 67.46) (end 173.361399 65.821399) (width 1.15) (layer B.Cu) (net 11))
 (segment (start 124.56 75.08) (end 127.1 75.08) (width 1.15) (layer B.Cu) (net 11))
 (segment (start 127.1 77.62) (end 132.25 72.47) (width 1.15) (layer F.Cu) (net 12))
 (segment (start 132.25 72.47) (end 132.25 70.5) (width 1.15) (layer F.Cu) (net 12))
 (segment (start 132.25 70.5) (end 138 64.75) (width 1.15) (layer F.Cu) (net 12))
 (segment (start 138 64.75) (end 174.71513 64.75) (width 1.15) (layer F.Cu) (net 12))
 (segment (start 174.71513 64.75) (end 177.5 67.53487) (width 1.15) (layer F.Cu) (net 12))
 (segment (start 177.5 67.53487) (end 177.5 71.5) (width 1.15) (layer F.Cu) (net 12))
 (segment (start 177.5 71.5) (end 176.46 72.54) (width 1.15) (layer F.Cu) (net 12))
 (segment (start 176.46 72.54) (end 175 72.54) (width 1.15) (layer F.Cu) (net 12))
 (segment (start 124.56 77.62) (end 127.1 77.62) (width 1.15) (layer F.Cu) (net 12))
 (segment (start 175 80.16) (end 177 82.16) (width 1.15) (layer F.Cu) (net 13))
 (segment (start 177 82.16) (end 177 85.66513) (width 1.15) (layer F.Cu) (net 13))
 (segment (start 177 85.66513) (end 174.91513 87.75) (width 1.15) (layer F.Cu) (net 13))
 (segment (start 174.91513 87.75) (end 148.5 87.75) (width 1.15) (layer F.Cu) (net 13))
 (segment (start 148.5 87.75) (end 140.25 79.5) (width 1.15) (layer F.Cu) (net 13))
 (segment (start 140.25 73.6164) (end 139.1736 72.54) (width 1.15) (layer F.Cu) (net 13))
 (segment (start 140.25 79.5) (end 140.25 73.6164) (width 1.15) (layer F.Cu) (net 13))
 (segment (start 139.1736 72.54) (end 137.16 72.54) (width 1.15) (layer F.Cu) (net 13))
 (segment (start 134.62 72.54) (end 137.16 72.54) (width 1.15) (layer F.Cu) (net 13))
 (segment (start 138.023599 75.943599) (end 137.16 75.08) (width 1.15) (layer B.Cu) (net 14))
 (segment (start 174.212196 86.878601) (end 148.958601 86.878601) (width 1.15) (layer B.Cu) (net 14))
 (segment (start 175 86.090798) (end 174.212196 86.878601) (width 1.15) (layer B.Cu) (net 14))
 (segment (start 175 85.24) (end 175 86.090798) (width 1.15) (layer B.Cu) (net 14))
 (segment (start 148.958601 86.878601) (end 138.023599 75.943599) (width 1.15) (layer B.Cu) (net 14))
 (segment (start 137.16 75.08) (end 134.62 75.08) (width 1.15) (layer B.Cu) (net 14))
 (segment (start 175 82.7) (end 176.75 84.45) (width 1.15) (layer B.Cu) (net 15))
 (segment (start 176.75 84.45) (end 176.75 86.25) (width 1.15) (layer B.Cu) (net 15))
 (segment (start 176.75 86.25) (end 174.771389 88.228612) (width 1.15) (layer B.Cu) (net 15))
 (segment (start 174.771389 88.228612) (end 147.768612 88.228612) (width 1.15) (layer B.Cu) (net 15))
 (segment (start 147.768612 88.228612) (end 137.16 77.62) (width 1.15) (layer B.Cu) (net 15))
 (segment (start 137.16 77.62) (end 134.62 77.62) (width 1.15) (layer B.Cu) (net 15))
 (segment (start 172.46 67.46) (end 150.2864 67.46) (width 1.15) (layer B.Cu) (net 16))
 (segment (start 150.2864 67.46) (end 147.22 70.5264) (width 1.15) (layer B.Cu) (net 16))
 (segment (start 147.22 70.5264) (end 147.22 72.54) (width 1.15) (layer B.Cu) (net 16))
 (segment (start 144.68 72.54) (end 147.22 72.54) (width 1.15) (layer B.Cu) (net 16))
 (segment (start 150.75 74) (end 149.67 75.08) (width 1.15) (layer B.Cu) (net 17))
 (segment (start 149.67 75.08) (end 147.22 75.08) (width 1.15) (layer B.Cu) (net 17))
 (segment (start 150.75 70) (end 150.75 74) (width 1.15) (layer B.Cu) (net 17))
 (segment (start 151.75 69) (end 150.75 70) (width 1.15) (layer B.Cu) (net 17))
 (segment (start 171.46 69) (end 151.75 69) (width 1.15) (layer B.Cu) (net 17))
 (segment (start 172.46 70) (end 171.46 69) (width 1.15) (layer B.Cu) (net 17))
 (segment (start 144.68 75.08) (end 147.22 75.08) (width 1.15) (layer B.Cu) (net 17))
 (segment (start 147.22 77.62) (end 144.68 77.62) (width 1.15) (layer B.Cu) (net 18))
 (segment (start 152.5 77.25) (end 152.13 77.62) (width 1.15) (layer B.Cu) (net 18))
 (segment (start 152.13 77.62) (end 147.22 77.62) (width 1.15) (layer B.Cu) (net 18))
 (segment (start 152.5 71.25) (end 152.5 77.25) (width 1.15) (layer B.Cu) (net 18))
 (segment (start 153.25 70.5) (end 152.5 71.25) (width 1.15) (layer B.Cu) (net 18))
 (segment (start 170.42 70.5) (end 153.25 70.5) (width 1.15) (layer B.Cu) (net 18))
 (segment (start 172.46 72.54) (end 170.42 70.5) (width 1.15) (layer B.Cu) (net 18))
 (segment (start 157.28 72.54) (end 154.74 72.54) (width 1.15) (layer B.Cu) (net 19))
 (segment (start 162.25 73.75) (end 161.04 72.54) (width 1.15) (layer B.Cu) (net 19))
 (segment (start 161.04 72.54) (end 157.28 72.54) (width 1.15) (layer B.Cu) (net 19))
 (segment (start 162.25 80.5) (end 162.25 73.75) (width 1.15) (layer B.Cu) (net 19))
 (segment (start 163.548601 81.798601) (end 162.25 80.5) (width 1.15) (layer B.Cu) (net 19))
 (segment (start 172.46 80.16) (end 170.821399 81.798601) (width 1.15) (layer B.Cu) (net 19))
 (segment (start 170.821399 81.798601) (end 163.548601 81.798601) (width 1.15) (layer B.Cu) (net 19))
 (segment (start 160.75 81) (end 163.313599 83.563599) (width 1.15) (layer B.Cu) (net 20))
 (segment (start 163.313599 83.563599) (end 171.596401 83.563599) (width 1.15) (layer B.Cu) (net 20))
 (segment (start 171.596401 83.563599) (end 172.46 82.7) (width 1.15) (layer B.Cu) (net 20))
 (segment (start 160.75 76.5) (end 160.75 81) (width 1.15) (layer B.Cu) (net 20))
 (segment (start 159.33 75.08) (end 160.75 76.5) (width 1.15) (layer B.Cu) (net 20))
 (segment (start 157.28 75.08) (end 159.33 75.08) (width 1.15) (layer B.Cu) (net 20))
 (segment (start 154.74 75.08) (end 157.28 75.08) (width 1.15) (layer B.Cu) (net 20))
 (segment (start 158.143599 78.483599) (end 157.28 77.62) (width 1.15) (layer B.Cu) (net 21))
 (segment (start 159.25 79.59) (end 158.143599 78.483599) (width 1.15) (layer B.Cu) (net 21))
 (segment (start 159.25 82.25) (end 159.25 79.59) (width 1.15) (layer B.Cu) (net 21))
 (segment (start 162.24 85.24) (end 159.25 82.25) (width 1.15) (layer B.Cu) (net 21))
 (segment (start 172.46 85.24) (end 162.24 85.24) (width 1.15) (layer B.Cu) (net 21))
 (segment (start 157.28 77.62) (end 154.74 77.62) (width 1.15) (layer B.Cu) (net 21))
 (segment (start 167.34 75.08) (end 172.46 75.08) (width 1.15) (layer B.Cu) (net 22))
 (segment (start 164.8 75.08) (end 167.34 75.08) (width 1.15) (layer B.Cu) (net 22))
 (segment (start 167.34 77.62) (end 172.46 77.62) (width 1.15) (layer B.Cu) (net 23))
 (segment (start 164.8 77.62) (end 167.34 77.62) (width 1.15) (layer B.Cu) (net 23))
 (segment (start 178.5 73.5) (end 176.92 75.08) (width 0.3) (layer F.Cu) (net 8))
 (segment (start 176.92 75.08) (end 175 75.08) (width 0.3) (layer F.Cu) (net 8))
 (segment (start 178.5 65.25) (end 178.5 73.5) (width 0.3) (layer F.Cu) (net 8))
 (segment (start 176.75 63.5) (end 178.5 65.25) (width 0.3) (layer F.Cu) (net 8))
 (segment (start 128.402798 63.5) (end 176.75 63.5) (width 0.3) (layer F.Cu) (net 8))
 (segment (start 120.576399 71.326399) (end 128.402798 63.5) (width 0.3) (layer F.Cu) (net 8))
 (segment (start 114.5 72.54) (end 115.713601 71.326399) (width 0.3) (layer F.Cu) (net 8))
 (segment (start 115.713601 71.326399) (end 120.576399 71.326399) (width 0.3) (layer F.Cu) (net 8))
 (segment (start 131.25 89) (end 118.543601 76.293601) (width 0.3) (layer F.Cu) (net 9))
 (segment (start 118.543601 76.293601) (end 115.713601 76.293601) (width 0.3) (layer F.Cu) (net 9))
 (segment (start 115.713601 76.293601) (end 115.363599 75.943599) (width 0.3) (layer F.Cu) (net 9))
 (segment (start 115.363599 75.943599) (end 114.5 75.08) (width 0.3) (layer F.Cu) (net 9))
 (segment (start 175.75 89) (end 131.25 89) (width 0.3) (layer F.Cu) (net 9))
 (segment (start 178.25 86.5) (end 175.75 89) (width 0.3) (layer F.Cu) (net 9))
 (segment (start 178.25 80.87) (end 178.25 86.5) (width 0.3) (layer F.Cu) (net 9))
 (segment (start 175 77.62) (end 178.25 80.87) (width 0.3) (layer F.Cu) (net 9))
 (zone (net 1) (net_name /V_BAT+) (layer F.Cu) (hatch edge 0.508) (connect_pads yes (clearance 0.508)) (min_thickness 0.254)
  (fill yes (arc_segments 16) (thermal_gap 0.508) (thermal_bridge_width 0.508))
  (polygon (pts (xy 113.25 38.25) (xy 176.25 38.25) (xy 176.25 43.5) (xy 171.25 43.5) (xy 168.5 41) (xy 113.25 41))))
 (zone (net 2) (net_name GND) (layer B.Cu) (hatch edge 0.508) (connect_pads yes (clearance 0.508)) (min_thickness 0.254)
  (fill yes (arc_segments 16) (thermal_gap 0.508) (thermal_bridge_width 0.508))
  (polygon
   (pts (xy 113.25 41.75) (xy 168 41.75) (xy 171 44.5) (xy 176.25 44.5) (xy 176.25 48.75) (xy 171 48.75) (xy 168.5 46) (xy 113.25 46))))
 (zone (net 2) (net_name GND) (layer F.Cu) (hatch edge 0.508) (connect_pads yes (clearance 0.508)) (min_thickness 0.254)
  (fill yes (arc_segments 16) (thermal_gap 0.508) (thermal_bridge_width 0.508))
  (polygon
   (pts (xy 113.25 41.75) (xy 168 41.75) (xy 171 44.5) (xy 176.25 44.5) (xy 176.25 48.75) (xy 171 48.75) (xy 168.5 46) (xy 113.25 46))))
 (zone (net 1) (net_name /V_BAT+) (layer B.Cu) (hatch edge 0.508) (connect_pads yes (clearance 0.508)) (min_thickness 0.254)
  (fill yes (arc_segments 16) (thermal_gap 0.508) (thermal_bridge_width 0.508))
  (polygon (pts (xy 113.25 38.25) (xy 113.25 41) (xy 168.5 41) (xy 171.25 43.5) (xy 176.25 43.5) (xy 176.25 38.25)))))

